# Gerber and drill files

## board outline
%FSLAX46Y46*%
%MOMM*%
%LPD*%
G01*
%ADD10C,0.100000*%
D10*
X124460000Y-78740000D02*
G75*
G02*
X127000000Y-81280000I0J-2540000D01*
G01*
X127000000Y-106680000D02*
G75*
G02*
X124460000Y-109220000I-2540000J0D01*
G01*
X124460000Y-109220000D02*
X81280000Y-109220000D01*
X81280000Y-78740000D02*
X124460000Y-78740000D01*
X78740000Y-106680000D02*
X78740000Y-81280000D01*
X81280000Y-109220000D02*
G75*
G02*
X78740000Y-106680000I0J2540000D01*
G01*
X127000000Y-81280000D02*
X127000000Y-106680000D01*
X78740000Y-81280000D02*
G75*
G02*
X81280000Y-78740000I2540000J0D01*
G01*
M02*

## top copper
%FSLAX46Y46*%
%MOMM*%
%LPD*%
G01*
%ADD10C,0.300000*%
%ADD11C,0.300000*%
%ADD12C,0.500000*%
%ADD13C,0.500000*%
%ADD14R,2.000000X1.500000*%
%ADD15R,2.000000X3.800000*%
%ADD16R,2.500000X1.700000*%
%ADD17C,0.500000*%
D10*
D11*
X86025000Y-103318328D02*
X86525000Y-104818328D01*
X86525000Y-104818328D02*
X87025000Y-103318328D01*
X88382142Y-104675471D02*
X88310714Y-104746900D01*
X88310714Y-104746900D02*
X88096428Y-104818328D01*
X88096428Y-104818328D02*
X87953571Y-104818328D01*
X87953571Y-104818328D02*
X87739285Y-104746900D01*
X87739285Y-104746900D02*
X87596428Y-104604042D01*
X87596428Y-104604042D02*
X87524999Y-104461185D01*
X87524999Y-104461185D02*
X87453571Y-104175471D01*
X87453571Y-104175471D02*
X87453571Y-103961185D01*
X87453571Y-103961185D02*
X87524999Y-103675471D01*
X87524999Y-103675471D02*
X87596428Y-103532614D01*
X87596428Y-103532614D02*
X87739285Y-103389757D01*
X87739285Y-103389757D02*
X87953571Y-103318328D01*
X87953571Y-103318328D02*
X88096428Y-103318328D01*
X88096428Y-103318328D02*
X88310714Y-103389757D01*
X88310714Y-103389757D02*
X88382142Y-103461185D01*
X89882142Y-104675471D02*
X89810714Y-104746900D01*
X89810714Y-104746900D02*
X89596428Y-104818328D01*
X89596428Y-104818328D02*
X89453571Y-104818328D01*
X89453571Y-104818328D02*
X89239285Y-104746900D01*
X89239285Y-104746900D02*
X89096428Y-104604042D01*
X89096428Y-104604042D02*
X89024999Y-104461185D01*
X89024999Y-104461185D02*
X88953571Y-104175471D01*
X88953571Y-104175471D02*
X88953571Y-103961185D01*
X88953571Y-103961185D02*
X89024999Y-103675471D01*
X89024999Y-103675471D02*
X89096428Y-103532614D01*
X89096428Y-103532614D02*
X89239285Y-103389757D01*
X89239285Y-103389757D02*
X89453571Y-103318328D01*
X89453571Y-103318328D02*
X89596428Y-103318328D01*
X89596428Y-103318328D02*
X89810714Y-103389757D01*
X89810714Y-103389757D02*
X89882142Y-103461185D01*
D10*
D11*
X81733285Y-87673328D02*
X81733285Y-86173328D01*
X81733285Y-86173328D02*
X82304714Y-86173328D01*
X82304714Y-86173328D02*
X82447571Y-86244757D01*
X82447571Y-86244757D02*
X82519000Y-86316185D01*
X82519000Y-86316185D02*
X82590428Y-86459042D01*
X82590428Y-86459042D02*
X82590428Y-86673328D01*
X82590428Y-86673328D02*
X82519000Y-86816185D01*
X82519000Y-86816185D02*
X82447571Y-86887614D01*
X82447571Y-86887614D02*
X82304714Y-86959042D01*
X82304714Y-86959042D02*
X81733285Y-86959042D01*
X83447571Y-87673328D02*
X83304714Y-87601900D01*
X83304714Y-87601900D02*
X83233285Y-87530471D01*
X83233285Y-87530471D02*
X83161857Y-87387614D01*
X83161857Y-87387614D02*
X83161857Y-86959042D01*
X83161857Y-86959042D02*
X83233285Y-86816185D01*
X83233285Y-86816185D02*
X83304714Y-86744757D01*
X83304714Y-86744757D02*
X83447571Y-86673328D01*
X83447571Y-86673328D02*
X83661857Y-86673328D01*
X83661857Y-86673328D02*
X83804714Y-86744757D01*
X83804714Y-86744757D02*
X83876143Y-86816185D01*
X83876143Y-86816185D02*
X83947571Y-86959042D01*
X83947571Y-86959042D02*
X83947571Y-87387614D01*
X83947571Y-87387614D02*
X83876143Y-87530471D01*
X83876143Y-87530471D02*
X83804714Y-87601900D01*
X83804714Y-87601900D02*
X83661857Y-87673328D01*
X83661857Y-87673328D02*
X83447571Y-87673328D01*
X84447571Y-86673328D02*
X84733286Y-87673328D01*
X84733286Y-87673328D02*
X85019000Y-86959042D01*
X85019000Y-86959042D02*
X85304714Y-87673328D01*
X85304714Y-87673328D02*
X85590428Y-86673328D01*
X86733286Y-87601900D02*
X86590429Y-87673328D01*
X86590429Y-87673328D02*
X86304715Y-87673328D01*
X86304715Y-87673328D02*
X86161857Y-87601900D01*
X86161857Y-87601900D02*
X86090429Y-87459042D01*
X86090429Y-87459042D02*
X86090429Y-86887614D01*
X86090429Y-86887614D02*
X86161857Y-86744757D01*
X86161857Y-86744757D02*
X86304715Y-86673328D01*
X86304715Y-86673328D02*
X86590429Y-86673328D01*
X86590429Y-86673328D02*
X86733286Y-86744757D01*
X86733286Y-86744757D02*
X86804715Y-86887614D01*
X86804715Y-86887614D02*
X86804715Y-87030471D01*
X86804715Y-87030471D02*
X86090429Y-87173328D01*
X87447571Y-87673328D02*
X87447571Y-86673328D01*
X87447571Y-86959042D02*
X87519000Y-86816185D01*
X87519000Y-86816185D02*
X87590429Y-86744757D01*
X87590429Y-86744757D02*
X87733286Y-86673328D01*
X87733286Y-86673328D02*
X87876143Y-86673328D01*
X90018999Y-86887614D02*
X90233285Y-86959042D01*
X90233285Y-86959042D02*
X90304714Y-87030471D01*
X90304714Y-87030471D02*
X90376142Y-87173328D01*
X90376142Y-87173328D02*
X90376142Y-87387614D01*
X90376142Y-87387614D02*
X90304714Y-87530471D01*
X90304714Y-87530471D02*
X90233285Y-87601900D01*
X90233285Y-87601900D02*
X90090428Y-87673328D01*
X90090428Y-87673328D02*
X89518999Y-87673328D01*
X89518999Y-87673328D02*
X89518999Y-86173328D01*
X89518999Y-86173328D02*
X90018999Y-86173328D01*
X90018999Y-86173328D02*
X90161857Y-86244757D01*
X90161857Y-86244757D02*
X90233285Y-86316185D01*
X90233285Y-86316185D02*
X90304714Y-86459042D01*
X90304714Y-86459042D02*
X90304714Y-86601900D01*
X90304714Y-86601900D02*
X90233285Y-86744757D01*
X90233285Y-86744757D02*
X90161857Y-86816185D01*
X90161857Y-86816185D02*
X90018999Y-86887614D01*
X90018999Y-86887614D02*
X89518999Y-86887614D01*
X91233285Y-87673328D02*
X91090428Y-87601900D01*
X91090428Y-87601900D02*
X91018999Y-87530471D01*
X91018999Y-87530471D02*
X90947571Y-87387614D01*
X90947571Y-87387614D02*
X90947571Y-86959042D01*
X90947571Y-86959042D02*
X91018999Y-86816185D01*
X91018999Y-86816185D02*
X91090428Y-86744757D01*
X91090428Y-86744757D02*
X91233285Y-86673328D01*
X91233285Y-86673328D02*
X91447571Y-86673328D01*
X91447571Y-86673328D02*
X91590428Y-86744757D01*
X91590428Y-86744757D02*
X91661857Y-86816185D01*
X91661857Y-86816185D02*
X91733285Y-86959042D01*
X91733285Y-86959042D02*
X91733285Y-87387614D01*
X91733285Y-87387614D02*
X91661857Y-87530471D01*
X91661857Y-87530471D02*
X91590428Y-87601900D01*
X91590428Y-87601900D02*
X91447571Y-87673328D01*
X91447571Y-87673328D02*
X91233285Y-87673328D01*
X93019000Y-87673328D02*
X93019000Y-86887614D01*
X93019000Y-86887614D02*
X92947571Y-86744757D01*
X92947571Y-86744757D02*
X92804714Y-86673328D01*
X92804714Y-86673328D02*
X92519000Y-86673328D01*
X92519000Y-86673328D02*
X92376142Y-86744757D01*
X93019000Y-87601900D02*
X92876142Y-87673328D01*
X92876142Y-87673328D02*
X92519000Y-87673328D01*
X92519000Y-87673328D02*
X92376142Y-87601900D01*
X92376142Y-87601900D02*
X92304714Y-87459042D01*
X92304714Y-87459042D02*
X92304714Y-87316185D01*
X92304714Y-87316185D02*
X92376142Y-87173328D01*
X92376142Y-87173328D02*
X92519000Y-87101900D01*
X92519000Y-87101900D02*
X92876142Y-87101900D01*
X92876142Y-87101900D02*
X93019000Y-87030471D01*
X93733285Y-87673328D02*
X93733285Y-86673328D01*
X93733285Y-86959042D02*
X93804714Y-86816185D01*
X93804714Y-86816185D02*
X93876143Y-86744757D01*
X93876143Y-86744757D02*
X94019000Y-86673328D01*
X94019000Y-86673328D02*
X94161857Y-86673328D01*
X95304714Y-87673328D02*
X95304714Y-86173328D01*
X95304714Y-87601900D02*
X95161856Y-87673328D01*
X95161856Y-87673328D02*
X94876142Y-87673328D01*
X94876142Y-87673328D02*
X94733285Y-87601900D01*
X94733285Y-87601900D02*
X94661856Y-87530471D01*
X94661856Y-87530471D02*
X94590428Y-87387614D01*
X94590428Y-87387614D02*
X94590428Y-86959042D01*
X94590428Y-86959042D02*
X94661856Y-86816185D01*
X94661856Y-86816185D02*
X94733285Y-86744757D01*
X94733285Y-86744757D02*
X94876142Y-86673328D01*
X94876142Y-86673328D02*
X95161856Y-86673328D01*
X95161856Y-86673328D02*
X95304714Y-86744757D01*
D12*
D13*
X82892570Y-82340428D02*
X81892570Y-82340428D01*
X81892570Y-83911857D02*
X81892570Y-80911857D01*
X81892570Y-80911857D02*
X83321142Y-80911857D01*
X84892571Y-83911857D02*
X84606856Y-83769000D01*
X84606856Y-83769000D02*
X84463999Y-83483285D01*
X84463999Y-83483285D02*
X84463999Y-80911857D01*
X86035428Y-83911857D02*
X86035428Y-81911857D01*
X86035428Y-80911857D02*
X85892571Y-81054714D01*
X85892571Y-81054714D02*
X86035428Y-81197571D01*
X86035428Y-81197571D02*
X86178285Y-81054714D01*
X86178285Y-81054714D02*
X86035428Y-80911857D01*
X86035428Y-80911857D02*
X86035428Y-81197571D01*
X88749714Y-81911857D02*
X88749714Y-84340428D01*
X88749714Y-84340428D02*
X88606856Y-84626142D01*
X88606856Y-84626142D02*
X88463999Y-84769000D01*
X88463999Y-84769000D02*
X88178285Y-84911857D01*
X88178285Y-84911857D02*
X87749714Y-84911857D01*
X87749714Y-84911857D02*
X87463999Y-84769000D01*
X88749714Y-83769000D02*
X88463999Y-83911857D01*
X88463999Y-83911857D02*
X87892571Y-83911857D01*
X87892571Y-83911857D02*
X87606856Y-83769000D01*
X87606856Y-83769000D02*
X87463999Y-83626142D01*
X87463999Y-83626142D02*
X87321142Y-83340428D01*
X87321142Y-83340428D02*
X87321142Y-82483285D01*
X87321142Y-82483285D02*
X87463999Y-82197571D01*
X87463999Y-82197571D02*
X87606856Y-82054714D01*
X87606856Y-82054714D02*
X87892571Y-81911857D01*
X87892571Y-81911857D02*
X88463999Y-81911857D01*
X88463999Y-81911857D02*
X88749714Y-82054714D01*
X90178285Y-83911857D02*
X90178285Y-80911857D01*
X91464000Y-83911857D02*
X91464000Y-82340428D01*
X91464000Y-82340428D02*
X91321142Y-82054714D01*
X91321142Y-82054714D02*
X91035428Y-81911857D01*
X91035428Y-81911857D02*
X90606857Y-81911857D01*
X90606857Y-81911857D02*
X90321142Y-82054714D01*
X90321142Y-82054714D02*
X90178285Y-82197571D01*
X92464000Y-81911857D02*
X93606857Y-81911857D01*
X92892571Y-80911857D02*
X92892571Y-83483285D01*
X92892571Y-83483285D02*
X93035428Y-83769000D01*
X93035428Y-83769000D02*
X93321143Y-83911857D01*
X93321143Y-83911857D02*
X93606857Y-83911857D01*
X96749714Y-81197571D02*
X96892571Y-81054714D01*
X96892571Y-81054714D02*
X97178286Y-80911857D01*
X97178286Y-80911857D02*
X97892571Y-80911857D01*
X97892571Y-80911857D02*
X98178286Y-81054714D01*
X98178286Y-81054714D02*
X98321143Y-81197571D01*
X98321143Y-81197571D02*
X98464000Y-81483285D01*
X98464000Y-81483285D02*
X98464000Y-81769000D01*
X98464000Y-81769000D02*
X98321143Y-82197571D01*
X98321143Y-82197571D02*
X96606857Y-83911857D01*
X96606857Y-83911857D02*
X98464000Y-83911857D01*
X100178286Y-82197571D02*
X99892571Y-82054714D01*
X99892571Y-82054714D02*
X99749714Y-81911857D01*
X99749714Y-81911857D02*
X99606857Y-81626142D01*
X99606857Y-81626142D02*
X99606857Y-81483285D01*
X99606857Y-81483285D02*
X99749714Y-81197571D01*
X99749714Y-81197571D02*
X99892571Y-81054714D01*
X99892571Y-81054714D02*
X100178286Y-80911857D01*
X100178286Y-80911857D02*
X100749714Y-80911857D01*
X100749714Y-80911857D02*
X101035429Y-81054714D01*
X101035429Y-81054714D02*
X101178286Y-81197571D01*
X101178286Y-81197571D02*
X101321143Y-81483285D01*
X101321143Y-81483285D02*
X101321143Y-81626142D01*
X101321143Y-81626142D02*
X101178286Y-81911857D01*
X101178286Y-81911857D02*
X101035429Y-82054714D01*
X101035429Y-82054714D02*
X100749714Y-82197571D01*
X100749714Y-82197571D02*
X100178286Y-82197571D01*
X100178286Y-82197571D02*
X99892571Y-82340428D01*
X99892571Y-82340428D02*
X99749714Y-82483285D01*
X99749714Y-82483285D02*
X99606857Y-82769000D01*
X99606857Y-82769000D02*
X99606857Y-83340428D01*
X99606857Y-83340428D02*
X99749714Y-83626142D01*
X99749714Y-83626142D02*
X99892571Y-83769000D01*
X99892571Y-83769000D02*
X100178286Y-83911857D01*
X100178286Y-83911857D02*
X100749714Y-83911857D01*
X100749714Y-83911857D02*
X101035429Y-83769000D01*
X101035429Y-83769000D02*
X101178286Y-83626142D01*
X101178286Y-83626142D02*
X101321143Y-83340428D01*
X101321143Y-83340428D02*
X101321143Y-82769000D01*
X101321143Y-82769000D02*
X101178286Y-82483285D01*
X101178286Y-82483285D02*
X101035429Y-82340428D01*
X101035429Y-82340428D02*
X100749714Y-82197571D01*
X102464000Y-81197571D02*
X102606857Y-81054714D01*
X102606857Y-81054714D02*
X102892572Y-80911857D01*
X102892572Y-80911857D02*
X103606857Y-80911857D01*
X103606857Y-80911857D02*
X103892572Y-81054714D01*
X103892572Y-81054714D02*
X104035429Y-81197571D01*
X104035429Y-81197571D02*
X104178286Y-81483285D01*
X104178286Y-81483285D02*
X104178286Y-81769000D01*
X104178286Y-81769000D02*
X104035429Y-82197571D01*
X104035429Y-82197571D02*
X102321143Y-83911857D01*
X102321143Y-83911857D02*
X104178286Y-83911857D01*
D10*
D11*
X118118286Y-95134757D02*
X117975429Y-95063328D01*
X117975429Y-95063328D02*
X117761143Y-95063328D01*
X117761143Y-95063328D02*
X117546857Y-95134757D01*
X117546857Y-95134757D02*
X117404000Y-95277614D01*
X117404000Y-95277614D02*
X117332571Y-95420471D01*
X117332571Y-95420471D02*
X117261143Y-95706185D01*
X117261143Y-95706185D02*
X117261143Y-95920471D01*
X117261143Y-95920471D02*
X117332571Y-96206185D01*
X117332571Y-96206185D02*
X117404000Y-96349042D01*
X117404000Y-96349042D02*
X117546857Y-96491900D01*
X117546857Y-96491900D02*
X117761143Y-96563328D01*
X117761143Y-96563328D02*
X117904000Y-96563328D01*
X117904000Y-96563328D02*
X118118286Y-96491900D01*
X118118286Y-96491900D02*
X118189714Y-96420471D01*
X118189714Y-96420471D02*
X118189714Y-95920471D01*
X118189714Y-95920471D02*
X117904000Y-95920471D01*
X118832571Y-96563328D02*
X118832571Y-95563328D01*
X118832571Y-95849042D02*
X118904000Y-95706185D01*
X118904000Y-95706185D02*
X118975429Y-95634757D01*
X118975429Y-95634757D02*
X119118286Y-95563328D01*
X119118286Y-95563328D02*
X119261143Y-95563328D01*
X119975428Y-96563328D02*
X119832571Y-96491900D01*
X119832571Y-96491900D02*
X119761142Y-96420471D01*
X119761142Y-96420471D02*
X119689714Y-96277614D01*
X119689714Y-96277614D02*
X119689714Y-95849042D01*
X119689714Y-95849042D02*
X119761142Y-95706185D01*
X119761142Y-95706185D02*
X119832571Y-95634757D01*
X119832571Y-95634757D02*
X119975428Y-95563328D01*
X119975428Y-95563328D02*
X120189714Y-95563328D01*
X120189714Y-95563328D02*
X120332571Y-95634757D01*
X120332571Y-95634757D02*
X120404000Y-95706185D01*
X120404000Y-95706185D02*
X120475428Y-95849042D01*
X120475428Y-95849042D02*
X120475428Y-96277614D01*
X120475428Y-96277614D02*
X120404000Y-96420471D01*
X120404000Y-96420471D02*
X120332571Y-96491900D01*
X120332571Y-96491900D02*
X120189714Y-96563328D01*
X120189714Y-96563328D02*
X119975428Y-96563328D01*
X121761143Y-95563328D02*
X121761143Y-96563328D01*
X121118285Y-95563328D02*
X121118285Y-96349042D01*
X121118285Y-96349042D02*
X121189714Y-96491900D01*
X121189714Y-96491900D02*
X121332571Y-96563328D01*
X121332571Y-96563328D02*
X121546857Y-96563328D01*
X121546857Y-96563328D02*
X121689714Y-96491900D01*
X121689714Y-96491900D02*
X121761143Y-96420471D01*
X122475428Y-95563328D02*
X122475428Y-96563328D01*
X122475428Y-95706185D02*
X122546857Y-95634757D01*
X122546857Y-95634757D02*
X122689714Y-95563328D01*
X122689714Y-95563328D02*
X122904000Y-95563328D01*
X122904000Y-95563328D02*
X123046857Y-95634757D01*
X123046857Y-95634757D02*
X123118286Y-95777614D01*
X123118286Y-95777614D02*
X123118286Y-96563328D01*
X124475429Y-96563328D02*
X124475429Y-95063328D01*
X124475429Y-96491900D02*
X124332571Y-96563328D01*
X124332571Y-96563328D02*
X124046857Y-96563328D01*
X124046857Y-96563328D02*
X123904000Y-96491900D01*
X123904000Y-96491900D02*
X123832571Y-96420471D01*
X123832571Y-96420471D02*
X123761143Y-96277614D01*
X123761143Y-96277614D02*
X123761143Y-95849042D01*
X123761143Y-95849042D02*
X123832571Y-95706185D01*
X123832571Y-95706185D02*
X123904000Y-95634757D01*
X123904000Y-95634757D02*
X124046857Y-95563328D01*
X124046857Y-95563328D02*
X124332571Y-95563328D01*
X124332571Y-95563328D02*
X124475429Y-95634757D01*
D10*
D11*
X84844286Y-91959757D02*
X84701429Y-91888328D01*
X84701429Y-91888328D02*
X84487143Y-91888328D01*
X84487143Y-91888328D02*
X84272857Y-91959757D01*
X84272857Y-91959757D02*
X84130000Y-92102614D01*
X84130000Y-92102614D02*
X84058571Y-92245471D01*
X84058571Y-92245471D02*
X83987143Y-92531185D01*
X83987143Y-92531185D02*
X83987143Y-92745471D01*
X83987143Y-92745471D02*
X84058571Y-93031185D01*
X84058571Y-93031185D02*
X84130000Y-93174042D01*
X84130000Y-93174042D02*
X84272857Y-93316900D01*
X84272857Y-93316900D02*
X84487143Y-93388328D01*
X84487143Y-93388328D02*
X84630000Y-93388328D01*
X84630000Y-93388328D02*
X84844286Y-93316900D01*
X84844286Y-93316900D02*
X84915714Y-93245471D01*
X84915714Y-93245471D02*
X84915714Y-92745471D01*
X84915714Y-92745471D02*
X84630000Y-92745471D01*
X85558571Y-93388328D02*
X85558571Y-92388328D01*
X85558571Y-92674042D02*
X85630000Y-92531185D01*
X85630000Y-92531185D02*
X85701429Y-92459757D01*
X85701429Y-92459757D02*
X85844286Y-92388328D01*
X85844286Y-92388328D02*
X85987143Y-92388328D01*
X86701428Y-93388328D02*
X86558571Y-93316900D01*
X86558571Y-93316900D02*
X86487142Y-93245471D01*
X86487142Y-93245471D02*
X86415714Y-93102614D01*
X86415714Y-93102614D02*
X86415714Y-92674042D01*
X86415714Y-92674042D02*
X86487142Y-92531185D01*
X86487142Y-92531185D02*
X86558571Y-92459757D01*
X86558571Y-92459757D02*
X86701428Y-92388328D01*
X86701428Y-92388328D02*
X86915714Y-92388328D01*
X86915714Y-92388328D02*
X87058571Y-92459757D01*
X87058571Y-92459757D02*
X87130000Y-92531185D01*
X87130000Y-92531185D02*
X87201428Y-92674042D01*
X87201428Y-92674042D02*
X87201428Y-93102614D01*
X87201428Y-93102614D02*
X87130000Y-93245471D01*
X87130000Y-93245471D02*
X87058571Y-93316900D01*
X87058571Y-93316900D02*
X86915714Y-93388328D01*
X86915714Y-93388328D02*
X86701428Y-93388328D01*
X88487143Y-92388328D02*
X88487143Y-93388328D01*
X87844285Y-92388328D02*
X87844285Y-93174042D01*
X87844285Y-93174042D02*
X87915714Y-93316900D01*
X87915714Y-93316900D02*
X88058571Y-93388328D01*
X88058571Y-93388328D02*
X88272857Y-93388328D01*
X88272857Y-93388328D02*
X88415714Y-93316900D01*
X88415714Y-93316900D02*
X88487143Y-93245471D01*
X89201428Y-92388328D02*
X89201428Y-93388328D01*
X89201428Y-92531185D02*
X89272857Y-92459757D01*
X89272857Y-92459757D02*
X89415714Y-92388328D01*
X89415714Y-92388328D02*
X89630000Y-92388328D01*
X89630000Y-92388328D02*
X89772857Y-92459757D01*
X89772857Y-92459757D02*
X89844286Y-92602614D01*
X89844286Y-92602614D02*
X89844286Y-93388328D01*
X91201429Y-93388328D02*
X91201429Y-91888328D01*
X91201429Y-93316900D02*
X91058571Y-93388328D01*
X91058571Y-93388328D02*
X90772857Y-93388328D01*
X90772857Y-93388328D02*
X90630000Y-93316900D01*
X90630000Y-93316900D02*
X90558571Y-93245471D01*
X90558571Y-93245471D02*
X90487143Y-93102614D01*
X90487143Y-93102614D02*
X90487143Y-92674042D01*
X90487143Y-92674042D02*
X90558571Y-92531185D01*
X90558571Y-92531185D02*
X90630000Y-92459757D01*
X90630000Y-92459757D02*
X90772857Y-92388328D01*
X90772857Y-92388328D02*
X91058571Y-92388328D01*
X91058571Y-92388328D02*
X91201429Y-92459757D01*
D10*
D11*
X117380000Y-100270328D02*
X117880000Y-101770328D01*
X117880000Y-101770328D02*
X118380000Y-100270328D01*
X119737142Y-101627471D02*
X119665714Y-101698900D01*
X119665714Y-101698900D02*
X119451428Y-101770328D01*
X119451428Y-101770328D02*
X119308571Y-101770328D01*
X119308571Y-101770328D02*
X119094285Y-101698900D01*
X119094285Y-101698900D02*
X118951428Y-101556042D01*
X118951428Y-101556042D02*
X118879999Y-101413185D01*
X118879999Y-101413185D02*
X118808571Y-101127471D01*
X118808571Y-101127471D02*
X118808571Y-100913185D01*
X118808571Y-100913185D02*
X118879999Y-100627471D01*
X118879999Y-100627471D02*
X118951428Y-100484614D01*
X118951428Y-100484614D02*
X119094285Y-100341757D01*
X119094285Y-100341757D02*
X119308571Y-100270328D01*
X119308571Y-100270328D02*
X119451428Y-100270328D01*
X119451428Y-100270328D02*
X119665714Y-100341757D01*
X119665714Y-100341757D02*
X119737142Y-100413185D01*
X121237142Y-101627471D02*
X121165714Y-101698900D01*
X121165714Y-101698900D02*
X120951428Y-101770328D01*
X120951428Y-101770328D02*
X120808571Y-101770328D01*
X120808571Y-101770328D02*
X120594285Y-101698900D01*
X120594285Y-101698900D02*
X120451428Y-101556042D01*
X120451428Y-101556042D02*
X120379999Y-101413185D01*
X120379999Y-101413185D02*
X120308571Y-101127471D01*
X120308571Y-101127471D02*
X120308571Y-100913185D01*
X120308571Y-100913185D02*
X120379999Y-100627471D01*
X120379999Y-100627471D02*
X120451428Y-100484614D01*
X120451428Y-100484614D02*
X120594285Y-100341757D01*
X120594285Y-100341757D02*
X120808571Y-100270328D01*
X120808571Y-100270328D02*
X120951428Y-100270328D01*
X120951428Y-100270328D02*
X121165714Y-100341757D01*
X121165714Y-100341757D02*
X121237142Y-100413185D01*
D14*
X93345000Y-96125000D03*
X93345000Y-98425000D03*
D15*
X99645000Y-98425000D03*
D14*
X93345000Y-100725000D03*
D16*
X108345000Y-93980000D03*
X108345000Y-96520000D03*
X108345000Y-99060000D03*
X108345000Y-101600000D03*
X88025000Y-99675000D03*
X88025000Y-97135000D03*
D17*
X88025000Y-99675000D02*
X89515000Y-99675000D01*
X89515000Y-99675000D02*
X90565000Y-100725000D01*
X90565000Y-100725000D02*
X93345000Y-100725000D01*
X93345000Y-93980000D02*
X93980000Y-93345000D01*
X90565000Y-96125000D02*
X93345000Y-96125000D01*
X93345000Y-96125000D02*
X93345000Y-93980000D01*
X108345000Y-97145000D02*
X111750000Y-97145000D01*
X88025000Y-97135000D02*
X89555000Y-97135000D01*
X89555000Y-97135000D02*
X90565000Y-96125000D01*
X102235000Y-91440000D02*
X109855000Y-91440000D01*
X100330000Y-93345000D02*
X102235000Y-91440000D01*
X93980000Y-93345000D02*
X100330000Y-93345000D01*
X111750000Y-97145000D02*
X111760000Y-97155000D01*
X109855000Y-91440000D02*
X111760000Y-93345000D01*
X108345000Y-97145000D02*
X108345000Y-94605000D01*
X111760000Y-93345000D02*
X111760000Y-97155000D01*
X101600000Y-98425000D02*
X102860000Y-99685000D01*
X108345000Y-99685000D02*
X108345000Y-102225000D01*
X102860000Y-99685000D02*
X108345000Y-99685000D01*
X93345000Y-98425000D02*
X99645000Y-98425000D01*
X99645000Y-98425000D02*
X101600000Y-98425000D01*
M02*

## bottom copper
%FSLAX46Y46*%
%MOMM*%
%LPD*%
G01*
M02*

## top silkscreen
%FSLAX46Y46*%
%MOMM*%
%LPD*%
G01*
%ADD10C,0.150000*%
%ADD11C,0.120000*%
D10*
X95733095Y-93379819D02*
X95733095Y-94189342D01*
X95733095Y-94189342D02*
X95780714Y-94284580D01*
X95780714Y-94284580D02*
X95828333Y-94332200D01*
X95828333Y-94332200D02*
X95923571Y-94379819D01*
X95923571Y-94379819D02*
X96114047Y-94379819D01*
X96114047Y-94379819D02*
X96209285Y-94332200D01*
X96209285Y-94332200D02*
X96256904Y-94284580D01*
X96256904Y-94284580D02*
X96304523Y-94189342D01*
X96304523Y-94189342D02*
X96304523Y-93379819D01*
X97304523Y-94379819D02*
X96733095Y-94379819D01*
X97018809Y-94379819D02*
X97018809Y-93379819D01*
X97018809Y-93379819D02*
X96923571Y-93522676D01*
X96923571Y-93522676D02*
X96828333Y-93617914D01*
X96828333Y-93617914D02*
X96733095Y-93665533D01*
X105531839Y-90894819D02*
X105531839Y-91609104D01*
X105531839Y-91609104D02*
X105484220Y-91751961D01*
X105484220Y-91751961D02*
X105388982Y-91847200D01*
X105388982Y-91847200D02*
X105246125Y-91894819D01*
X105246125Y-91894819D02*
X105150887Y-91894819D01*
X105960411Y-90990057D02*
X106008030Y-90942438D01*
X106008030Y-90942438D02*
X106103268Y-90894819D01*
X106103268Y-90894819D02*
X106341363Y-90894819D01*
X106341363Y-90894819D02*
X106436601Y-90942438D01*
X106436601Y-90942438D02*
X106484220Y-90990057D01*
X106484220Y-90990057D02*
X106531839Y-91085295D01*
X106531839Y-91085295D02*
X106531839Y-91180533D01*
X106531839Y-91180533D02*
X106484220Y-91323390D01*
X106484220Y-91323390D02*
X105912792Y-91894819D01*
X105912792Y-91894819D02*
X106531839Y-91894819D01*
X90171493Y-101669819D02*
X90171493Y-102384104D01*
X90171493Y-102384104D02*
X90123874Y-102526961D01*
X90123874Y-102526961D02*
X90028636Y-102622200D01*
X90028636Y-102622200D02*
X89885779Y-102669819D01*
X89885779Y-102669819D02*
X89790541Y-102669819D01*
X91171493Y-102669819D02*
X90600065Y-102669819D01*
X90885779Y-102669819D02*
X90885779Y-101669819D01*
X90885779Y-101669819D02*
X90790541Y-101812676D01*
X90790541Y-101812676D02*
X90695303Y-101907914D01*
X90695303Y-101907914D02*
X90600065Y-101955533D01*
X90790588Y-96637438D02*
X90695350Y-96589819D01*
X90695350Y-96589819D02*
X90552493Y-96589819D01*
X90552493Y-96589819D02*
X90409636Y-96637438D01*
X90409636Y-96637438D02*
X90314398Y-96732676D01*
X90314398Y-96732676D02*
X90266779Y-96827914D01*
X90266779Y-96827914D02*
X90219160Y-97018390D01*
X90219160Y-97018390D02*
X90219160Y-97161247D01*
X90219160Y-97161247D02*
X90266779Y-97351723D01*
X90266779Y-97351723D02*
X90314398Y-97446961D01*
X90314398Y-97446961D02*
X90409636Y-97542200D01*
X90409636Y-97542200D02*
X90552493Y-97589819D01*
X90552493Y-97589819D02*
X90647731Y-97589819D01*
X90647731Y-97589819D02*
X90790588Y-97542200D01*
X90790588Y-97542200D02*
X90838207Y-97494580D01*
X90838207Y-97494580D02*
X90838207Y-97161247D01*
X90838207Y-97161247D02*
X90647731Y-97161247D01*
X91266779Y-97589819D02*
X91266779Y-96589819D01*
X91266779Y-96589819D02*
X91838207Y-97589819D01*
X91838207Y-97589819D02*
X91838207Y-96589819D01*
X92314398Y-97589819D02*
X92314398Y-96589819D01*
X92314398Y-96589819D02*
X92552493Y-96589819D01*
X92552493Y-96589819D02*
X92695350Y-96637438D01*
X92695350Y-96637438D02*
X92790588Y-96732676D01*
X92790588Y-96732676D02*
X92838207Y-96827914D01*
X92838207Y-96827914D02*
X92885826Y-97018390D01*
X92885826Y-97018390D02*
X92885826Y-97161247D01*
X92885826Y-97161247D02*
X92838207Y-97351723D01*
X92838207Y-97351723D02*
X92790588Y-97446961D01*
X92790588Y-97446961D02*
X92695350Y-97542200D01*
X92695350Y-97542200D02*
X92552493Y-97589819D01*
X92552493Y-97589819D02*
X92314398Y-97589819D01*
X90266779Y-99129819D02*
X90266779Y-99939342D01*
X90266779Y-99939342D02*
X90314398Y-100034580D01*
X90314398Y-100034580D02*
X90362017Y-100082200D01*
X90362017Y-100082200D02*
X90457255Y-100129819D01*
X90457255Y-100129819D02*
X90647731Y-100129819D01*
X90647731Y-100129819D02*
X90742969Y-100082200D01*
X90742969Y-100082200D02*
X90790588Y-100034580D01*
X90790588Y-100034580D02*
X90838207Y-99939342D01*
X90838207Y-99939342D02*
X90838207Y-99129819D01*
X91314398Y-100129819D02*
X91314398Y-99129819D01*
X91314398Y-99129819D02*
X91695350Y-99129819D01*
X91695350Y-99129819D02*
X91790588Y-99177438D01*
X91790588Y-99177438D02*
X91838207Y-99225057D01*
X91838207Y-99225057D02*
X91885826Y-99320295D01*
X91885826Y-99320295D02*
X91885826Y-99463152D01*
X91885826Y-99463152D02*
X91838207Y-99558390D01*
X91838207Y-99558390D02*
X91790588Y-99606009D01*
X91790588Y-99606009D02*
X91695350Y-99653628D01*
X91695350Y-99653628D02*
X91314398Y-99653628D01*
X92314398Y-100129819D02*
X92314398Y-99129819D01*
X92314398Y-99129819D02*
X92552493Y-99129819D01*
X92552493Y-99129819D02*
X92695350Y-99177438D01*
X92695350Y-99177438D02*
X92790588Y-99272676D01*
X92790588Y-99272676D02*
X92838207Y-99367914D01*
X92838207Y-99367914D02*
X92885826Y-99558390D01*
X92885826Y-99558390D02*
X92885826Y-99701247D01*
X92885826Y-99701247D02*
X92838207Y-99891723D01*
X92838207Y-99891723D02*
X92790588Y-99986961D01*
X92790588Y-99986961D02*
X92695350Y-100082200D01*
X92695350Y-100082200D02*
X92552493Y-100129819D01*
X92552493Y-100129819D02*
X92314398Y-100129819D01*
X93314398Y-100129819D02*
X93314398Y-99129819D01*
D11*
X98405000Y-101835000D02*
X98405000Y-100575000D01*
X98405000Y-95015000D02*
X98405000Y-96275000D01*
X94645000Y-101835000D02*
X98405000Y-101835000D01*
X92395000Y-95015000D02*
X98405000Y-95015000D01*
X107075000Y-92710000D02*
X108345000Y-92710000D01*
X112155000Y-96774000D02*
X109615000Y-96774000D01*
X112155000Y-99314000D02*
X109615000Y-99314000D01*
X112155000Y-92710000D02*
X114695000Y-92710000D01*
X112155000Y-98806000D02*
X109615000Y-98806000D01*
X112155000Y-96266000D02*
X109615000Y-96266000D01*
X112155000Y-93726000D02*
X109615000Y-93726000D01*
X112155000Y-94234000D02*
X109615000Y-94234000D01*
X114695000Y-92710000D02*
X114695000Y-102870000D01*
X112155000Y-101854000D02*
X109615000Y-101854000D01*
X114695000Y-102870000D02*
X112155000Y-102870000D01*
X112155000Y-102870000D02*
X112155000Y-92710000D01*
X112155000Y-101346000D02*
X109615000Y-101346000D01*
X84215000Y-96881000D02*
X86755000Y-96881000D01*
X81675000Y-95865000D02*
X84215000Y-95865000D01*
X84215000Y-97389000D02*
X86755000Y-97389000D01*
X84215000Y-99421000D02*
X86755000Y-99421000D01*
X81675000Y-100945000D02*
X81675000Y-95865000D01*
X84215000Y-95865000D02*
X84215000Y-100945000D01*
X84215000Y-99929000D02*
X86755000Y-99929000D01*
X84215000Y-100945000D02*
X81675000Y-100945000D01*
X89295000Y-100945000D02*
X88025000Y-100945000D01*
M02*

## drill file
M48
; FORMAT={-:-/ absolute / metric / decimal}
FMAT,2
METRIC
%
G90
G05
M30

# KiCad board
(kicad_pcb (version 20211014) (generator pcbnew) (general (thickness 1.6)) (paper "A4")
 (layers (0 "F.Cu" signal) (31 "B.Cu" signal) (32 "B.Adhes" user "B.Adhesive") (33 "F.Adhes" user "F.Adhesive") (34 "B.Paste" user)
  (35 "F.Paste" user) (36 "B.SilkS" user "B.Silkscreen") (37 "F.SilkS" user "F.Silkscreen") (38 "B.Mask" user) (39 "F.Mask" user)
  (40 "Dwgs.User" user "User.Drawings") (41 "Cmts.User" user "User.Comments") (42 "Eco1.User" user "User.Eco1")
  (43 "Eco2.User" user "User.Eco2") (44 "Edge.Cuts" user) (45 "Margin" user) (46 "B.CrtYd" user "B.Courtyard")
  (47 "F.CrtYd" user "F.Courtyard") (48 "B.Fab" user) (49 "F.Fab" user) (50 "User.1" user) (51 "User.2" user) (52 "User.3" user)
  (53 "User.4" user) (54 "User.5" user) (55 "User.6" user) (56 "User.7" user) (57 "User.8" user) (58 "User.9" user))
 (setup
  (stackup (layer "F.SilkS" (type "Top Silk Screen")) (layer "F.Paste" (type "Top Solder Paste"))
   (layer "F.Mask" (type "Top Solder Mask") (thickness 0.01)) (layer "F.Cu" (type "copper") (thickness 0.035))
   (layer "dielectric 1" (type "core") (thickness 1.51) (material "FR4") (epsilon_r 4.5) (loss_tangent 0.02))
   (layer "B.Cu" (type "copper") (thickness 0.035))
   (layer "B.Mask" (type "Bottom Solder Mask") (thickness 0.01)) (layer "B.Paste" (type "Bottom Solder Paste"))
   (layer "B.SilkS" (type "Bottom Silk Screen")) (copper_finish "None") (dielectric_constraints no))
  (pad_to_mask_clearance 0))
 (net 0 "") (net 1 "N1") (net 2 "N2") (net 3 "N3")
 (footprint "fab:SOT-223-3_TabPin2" (layer "F.Cu") (at 96.495 98.425)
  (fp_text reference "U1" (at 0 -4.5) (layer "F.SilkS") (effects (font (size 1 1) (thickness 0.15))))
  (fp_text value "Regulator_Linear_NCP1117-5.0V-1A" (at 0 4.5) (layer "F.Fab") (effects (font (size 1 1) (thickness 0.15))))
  (fp_line (start 1.91 3.41) (end 1.91 2.15) (layer "F.SilkS") (width 0.12))
  (fp_line (start 1.91 -3.41) (end 1.91 -2.15) (layer "F.SilkS") (width 0.12))
  (fp_line (start -1.85 3.41) (end 1.91 3.41) (layer "F.SilkS") (width 0.12))
  (fp_line (start -4.1 -3.41) (end 1.91 -3.41) (layer "F.SilkS") (width 0.12))
  (pad "1" smd rect locked (at -3.15 -2.3) (size 2 1.5) (layers "F.Cu" "F.Paste" "F.Mask") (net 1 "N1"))
  (pad "2" smd rect locked (at -3.15 0) (size 2 1.5) (layers "F.Cu" "F.Paste" "F.Mask") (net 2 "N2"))
  (pad "2" smd rect locked (at 3.15 0) (size 2 3.8) (layers "F.Cu" "F.Paste" "F.Mask") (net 2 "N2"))
  (pad "3" smd rect locked (at -3.15 2.3) (size 2 1.5) (layers "F.Cu" "F.Paste" "F.Mask") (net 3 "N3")))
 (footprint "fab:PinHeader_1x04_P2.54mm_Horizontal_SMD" (layer "F.Cu") (at 108.345 93.98)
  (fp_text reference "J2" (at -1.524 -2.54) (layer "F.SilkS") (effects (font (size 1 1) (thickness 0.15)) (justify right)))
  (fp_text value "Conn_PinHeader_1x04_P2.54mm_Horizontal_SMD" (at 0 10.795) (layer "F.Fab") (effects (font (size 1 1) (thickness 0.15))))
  (fp_line (start -1.27 -1.27) (end 0 -1.27) (layer "F.SilkS") (width 0.12))
  (fp_line (start 3.81 2.794) (end 1.27 2.794) (layer "F.SilkS") (width 0.12))
  (fp_line (start 3.81 5.334) (end 1.27 5.334) (layer "F.SilkS") (width 0.12))
  (fp_line (start 3.81 -1.27) (end 6.35 -1.27) (layer "F.SilkS") (width 0.12))
  (fp_line (start 3.81 4.826) (end 1.27 4.826) (layer "F.SilkS") (width 0.12))
  (fp_line (start 3.81 2.286) (end 1.27 2.286) (layer "F.SilkS") (width 0.12))
  (fp_line (start 3.81 -0.254) (end 1.27 -0.254) (layer "F.SilkS") (width 0.12))
  (fp_line (start 3.81 0.254) (end 1.27 0.254) (layer "F.SilkS") (width 0.12))
  (fp_line (start 6.35 -1.27) (end 6.35 8.89) (layer "F.SilkS") (width 0.12))
  (fp_line (start 3.81 7.874) (end 1.27 7.874) (layer "F.SilkS") (width 0.12))
  (fp_line (start 6.35 8.89) (end 3.81 8.89) (layer "F.SilkS") (width 0.12))
  (fp_line (start 3.81 8.89) (end 3.81 -1.27) (layer "F.SilkS") (width 0.12))
  (fp_line (start 3.81 7.366) (end 1.27 7.366) (layer "F.SilkS") (width 0.12))
  (pad "1" smd rect locked (at 0 0) (size 2.5 1.7) (layers "F.Cu" "F.Paste" "F.Mask") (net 1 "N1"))
  (pad "2" smd rect locked (at 0 2.54) (size 2.5 1.7) (layers "F.Cu" "F.Paste" "F.Mask") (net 1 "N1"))
  (pad "3" smd rect locked (at 0 5.08) (size 2.5 1.7) (layers "F.Cu" "F.Paste" "F.Mask") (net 2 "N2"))
  (pad "4" smd rect locked (at 0 7.62) (size 2.5 1.7) (layers "F.Cu" "F.Paste" "F.Mask") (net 2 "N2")))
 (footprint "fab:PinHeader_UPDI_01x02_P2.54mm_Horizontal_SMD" (layer "F.Cu") (at 88.025 99.675 180)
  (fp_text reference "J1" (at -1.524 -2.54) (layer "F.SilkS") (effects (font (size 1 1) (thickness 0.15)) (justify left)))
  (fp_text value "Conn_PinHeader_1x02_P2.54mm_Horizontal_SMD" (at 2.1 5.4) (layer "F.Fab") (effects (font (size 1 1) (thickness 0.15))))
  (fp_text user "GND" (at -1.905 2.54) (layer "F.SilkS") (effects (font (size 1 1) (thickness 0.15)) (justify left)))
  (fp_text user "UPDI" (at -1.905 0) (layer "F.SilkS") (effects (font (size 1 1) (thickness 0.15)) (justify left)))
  (fp_line (start 3.81 2.794) (end 1.27 2.794) (layer "F.SilkS") (width 0.12))
  (fp_line (start 6.35 3.81) (end 3.81 3.81) (layer "F.SilkS") (width 0.12))
  (fp_line (start 3.81 2.286) (end 1.27 2.286) (layer "F.SilkS") (width 0.12))
  (fp_line (start 3.81 0.254) (end 1.27 0.254) (layer "F.SilkS") (width 0.12))
  (fp_line (start 6.35 -1.27) (end 6.35 3.81) (layer "F.SilkS") (width 0.12))
  (fp_line (start 3.81 3.81) (end 3.81 -1.27) (layer "F.SilkS") (width 0.12))
  (fp_line (start 3.81 -0.254) (end 1.27 -0.254) (layer "F.SilkS") (width 0.12))
  (fp_line (start 3.81 -1.27) (end 6.35 -1.27) (layer "F.SilkS") (width 0.12))
  (fp_line (start -1.27 -1.27) (end 0 -1.27) (layer "F.SilkS") (width 0.12))
  (pad "1" smd rect locked (at 0 0 180) (size 2.5 1.7) (layers "F.Cu" "F.Paste" "F.Mask") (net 3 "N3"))
  (pad "2" smd rect locked (at 0 2.54 180) (size 2.5 1.7) (layers "F.Cu" "F.Paste" "F.Mask") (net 1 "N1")))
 (gr_arc (start 124.46 78.74) (mid 126.256051 79.483949) (end 127 81.28) (layer "Edge.Cuts") (width 0.1))
 (gr_arc (start 127 106.68) (mid 126.256051 108.476051) (end 124.46 109.22) (layer "Edge.Cuts") (width 0.1))
 (gr_line (start 124.46 109.22) (end 81.28 109.22) (layer "Edge.Cuts") (width 0.1))
 (gr_line (start 81.28 78.74) (end 124.46 78.74) (layer "Edge.Cuts") (width 0.1))
 (gr_line (start 78.74 106.68) (end 78.74 81.28) (layer "Edge.Cuts") (width 0.1))
 (gr_arc (start 81.28 109.22) (mid 79.483949 108.476051) (end 78.74 106.68) (layer "Edge.Cuts") (width 0.1))
 (gr_line (start 127 81.28) (end 127 106.68) (layer "Edge.Cuts") (width 0.1))
 (gr_arc (start 78.74 81.28) (mid 79.483949 79.483949) (end 81.28 78.74) (layer "Edge.Cuts") (width 0.1))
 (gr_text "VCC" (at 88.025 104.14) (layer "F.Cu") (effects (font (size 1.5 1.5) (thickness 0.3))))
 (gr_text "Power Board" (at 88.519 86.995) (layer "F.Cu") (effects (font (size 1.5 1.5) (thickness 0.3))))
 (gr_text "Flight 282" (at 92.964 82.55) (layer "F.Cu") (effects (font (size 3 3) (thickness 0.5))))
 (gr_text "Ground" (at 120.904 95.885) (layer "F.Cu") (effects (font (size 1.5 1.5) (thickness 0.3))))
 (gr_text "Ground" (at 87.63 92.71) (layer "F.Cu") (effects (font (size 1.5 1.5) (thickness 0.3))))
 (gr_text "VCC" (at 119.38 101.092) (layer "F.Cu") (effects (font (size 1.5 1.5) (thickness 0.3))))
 (segment (start 88.025 99.675) (end 89.515 99.675) (width 0.5) (layer "F.Cu") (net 3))
 (segment (start 89.515 99.675) (end 90.565 100.725) (width 0.5) (layer "F.Cu") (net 3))
 (segment (start 90.565 100.725) (end 93.345 100.725) (width 0.5) (layer "F.Cu") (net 3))
 (segment (start 93.345 93.98) (end 93.98 93.345) (width 0.5) (layer "F.Cu") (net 1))
 (segment (start 90.565 96.125) (end 93.345 96.125) (width 0.5) (layer "F.Cu") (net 1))
 (segment (start 93.345 96.125) (end 93.345 93.98) (width 0.5) (layer "F.Cu") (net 1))
 (segment (start 108.345 97.145) (end 111.75 97.145) (width 0.5) (layer "F.Cu") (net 1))
 (segment (start 88.025 97.135) (end 89.555 97.135) (width 0.5) (layer "F.Cu") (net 1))
 (segment (start 89.555 97.135) (end 90.565 96.125) (width 0.5) (layer "F.Cu") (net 1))
 (segment (start 102.235 91.44) (end 109.855 91.44) (width 0.5) (layer "F.Cu") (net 1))
 (segment (start 100.33 93.345) (end 102.235 91.44) (width 0.5) (layer "F.Cu") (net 1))
 (segment (start 93.98 93.345) (end 100.33 93.345) (width 0.5) (layer "F.Cu") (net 1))
 (segment (start 111.75 97.145) (end 111.76 97.155) (width 0.5) (layer "F.Cu") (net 1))
 (segment (start 109.855 91.44) (end 111.76 93.345) (width 0.5) (layer "F.Cu") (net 1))
 (segment (start 108.345 97.145) (end 108.345 94.605) (width 0.5) (layer "F.Cu") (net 1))
 (segment (start 111.76 93.345) (end 111.76 97.155) (width 0.5) (layer "F.Cu") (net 1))
 (segment (start 101.6 98.425) (end 102.86 99.685) (width 0.5) (layer "F.Cu") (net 2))
 (segment (start 108.345 99.685) (end 108.345 102.225) (width 0.5) (layer "F.Cu") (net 2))
 (segment (start 102.86 99.685) (end 108.345 99.685) (width 0.5) (layer "F.Cu") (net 2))
 (segment (start 93.345 98.425) (end 99.645 98.425) (width 0.5) (layer "F.Cu") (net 2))
 (segment (start 99.645 98.425) (end 101.6 98.425) (width 0.5) (layer "F.Cu") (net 2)))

